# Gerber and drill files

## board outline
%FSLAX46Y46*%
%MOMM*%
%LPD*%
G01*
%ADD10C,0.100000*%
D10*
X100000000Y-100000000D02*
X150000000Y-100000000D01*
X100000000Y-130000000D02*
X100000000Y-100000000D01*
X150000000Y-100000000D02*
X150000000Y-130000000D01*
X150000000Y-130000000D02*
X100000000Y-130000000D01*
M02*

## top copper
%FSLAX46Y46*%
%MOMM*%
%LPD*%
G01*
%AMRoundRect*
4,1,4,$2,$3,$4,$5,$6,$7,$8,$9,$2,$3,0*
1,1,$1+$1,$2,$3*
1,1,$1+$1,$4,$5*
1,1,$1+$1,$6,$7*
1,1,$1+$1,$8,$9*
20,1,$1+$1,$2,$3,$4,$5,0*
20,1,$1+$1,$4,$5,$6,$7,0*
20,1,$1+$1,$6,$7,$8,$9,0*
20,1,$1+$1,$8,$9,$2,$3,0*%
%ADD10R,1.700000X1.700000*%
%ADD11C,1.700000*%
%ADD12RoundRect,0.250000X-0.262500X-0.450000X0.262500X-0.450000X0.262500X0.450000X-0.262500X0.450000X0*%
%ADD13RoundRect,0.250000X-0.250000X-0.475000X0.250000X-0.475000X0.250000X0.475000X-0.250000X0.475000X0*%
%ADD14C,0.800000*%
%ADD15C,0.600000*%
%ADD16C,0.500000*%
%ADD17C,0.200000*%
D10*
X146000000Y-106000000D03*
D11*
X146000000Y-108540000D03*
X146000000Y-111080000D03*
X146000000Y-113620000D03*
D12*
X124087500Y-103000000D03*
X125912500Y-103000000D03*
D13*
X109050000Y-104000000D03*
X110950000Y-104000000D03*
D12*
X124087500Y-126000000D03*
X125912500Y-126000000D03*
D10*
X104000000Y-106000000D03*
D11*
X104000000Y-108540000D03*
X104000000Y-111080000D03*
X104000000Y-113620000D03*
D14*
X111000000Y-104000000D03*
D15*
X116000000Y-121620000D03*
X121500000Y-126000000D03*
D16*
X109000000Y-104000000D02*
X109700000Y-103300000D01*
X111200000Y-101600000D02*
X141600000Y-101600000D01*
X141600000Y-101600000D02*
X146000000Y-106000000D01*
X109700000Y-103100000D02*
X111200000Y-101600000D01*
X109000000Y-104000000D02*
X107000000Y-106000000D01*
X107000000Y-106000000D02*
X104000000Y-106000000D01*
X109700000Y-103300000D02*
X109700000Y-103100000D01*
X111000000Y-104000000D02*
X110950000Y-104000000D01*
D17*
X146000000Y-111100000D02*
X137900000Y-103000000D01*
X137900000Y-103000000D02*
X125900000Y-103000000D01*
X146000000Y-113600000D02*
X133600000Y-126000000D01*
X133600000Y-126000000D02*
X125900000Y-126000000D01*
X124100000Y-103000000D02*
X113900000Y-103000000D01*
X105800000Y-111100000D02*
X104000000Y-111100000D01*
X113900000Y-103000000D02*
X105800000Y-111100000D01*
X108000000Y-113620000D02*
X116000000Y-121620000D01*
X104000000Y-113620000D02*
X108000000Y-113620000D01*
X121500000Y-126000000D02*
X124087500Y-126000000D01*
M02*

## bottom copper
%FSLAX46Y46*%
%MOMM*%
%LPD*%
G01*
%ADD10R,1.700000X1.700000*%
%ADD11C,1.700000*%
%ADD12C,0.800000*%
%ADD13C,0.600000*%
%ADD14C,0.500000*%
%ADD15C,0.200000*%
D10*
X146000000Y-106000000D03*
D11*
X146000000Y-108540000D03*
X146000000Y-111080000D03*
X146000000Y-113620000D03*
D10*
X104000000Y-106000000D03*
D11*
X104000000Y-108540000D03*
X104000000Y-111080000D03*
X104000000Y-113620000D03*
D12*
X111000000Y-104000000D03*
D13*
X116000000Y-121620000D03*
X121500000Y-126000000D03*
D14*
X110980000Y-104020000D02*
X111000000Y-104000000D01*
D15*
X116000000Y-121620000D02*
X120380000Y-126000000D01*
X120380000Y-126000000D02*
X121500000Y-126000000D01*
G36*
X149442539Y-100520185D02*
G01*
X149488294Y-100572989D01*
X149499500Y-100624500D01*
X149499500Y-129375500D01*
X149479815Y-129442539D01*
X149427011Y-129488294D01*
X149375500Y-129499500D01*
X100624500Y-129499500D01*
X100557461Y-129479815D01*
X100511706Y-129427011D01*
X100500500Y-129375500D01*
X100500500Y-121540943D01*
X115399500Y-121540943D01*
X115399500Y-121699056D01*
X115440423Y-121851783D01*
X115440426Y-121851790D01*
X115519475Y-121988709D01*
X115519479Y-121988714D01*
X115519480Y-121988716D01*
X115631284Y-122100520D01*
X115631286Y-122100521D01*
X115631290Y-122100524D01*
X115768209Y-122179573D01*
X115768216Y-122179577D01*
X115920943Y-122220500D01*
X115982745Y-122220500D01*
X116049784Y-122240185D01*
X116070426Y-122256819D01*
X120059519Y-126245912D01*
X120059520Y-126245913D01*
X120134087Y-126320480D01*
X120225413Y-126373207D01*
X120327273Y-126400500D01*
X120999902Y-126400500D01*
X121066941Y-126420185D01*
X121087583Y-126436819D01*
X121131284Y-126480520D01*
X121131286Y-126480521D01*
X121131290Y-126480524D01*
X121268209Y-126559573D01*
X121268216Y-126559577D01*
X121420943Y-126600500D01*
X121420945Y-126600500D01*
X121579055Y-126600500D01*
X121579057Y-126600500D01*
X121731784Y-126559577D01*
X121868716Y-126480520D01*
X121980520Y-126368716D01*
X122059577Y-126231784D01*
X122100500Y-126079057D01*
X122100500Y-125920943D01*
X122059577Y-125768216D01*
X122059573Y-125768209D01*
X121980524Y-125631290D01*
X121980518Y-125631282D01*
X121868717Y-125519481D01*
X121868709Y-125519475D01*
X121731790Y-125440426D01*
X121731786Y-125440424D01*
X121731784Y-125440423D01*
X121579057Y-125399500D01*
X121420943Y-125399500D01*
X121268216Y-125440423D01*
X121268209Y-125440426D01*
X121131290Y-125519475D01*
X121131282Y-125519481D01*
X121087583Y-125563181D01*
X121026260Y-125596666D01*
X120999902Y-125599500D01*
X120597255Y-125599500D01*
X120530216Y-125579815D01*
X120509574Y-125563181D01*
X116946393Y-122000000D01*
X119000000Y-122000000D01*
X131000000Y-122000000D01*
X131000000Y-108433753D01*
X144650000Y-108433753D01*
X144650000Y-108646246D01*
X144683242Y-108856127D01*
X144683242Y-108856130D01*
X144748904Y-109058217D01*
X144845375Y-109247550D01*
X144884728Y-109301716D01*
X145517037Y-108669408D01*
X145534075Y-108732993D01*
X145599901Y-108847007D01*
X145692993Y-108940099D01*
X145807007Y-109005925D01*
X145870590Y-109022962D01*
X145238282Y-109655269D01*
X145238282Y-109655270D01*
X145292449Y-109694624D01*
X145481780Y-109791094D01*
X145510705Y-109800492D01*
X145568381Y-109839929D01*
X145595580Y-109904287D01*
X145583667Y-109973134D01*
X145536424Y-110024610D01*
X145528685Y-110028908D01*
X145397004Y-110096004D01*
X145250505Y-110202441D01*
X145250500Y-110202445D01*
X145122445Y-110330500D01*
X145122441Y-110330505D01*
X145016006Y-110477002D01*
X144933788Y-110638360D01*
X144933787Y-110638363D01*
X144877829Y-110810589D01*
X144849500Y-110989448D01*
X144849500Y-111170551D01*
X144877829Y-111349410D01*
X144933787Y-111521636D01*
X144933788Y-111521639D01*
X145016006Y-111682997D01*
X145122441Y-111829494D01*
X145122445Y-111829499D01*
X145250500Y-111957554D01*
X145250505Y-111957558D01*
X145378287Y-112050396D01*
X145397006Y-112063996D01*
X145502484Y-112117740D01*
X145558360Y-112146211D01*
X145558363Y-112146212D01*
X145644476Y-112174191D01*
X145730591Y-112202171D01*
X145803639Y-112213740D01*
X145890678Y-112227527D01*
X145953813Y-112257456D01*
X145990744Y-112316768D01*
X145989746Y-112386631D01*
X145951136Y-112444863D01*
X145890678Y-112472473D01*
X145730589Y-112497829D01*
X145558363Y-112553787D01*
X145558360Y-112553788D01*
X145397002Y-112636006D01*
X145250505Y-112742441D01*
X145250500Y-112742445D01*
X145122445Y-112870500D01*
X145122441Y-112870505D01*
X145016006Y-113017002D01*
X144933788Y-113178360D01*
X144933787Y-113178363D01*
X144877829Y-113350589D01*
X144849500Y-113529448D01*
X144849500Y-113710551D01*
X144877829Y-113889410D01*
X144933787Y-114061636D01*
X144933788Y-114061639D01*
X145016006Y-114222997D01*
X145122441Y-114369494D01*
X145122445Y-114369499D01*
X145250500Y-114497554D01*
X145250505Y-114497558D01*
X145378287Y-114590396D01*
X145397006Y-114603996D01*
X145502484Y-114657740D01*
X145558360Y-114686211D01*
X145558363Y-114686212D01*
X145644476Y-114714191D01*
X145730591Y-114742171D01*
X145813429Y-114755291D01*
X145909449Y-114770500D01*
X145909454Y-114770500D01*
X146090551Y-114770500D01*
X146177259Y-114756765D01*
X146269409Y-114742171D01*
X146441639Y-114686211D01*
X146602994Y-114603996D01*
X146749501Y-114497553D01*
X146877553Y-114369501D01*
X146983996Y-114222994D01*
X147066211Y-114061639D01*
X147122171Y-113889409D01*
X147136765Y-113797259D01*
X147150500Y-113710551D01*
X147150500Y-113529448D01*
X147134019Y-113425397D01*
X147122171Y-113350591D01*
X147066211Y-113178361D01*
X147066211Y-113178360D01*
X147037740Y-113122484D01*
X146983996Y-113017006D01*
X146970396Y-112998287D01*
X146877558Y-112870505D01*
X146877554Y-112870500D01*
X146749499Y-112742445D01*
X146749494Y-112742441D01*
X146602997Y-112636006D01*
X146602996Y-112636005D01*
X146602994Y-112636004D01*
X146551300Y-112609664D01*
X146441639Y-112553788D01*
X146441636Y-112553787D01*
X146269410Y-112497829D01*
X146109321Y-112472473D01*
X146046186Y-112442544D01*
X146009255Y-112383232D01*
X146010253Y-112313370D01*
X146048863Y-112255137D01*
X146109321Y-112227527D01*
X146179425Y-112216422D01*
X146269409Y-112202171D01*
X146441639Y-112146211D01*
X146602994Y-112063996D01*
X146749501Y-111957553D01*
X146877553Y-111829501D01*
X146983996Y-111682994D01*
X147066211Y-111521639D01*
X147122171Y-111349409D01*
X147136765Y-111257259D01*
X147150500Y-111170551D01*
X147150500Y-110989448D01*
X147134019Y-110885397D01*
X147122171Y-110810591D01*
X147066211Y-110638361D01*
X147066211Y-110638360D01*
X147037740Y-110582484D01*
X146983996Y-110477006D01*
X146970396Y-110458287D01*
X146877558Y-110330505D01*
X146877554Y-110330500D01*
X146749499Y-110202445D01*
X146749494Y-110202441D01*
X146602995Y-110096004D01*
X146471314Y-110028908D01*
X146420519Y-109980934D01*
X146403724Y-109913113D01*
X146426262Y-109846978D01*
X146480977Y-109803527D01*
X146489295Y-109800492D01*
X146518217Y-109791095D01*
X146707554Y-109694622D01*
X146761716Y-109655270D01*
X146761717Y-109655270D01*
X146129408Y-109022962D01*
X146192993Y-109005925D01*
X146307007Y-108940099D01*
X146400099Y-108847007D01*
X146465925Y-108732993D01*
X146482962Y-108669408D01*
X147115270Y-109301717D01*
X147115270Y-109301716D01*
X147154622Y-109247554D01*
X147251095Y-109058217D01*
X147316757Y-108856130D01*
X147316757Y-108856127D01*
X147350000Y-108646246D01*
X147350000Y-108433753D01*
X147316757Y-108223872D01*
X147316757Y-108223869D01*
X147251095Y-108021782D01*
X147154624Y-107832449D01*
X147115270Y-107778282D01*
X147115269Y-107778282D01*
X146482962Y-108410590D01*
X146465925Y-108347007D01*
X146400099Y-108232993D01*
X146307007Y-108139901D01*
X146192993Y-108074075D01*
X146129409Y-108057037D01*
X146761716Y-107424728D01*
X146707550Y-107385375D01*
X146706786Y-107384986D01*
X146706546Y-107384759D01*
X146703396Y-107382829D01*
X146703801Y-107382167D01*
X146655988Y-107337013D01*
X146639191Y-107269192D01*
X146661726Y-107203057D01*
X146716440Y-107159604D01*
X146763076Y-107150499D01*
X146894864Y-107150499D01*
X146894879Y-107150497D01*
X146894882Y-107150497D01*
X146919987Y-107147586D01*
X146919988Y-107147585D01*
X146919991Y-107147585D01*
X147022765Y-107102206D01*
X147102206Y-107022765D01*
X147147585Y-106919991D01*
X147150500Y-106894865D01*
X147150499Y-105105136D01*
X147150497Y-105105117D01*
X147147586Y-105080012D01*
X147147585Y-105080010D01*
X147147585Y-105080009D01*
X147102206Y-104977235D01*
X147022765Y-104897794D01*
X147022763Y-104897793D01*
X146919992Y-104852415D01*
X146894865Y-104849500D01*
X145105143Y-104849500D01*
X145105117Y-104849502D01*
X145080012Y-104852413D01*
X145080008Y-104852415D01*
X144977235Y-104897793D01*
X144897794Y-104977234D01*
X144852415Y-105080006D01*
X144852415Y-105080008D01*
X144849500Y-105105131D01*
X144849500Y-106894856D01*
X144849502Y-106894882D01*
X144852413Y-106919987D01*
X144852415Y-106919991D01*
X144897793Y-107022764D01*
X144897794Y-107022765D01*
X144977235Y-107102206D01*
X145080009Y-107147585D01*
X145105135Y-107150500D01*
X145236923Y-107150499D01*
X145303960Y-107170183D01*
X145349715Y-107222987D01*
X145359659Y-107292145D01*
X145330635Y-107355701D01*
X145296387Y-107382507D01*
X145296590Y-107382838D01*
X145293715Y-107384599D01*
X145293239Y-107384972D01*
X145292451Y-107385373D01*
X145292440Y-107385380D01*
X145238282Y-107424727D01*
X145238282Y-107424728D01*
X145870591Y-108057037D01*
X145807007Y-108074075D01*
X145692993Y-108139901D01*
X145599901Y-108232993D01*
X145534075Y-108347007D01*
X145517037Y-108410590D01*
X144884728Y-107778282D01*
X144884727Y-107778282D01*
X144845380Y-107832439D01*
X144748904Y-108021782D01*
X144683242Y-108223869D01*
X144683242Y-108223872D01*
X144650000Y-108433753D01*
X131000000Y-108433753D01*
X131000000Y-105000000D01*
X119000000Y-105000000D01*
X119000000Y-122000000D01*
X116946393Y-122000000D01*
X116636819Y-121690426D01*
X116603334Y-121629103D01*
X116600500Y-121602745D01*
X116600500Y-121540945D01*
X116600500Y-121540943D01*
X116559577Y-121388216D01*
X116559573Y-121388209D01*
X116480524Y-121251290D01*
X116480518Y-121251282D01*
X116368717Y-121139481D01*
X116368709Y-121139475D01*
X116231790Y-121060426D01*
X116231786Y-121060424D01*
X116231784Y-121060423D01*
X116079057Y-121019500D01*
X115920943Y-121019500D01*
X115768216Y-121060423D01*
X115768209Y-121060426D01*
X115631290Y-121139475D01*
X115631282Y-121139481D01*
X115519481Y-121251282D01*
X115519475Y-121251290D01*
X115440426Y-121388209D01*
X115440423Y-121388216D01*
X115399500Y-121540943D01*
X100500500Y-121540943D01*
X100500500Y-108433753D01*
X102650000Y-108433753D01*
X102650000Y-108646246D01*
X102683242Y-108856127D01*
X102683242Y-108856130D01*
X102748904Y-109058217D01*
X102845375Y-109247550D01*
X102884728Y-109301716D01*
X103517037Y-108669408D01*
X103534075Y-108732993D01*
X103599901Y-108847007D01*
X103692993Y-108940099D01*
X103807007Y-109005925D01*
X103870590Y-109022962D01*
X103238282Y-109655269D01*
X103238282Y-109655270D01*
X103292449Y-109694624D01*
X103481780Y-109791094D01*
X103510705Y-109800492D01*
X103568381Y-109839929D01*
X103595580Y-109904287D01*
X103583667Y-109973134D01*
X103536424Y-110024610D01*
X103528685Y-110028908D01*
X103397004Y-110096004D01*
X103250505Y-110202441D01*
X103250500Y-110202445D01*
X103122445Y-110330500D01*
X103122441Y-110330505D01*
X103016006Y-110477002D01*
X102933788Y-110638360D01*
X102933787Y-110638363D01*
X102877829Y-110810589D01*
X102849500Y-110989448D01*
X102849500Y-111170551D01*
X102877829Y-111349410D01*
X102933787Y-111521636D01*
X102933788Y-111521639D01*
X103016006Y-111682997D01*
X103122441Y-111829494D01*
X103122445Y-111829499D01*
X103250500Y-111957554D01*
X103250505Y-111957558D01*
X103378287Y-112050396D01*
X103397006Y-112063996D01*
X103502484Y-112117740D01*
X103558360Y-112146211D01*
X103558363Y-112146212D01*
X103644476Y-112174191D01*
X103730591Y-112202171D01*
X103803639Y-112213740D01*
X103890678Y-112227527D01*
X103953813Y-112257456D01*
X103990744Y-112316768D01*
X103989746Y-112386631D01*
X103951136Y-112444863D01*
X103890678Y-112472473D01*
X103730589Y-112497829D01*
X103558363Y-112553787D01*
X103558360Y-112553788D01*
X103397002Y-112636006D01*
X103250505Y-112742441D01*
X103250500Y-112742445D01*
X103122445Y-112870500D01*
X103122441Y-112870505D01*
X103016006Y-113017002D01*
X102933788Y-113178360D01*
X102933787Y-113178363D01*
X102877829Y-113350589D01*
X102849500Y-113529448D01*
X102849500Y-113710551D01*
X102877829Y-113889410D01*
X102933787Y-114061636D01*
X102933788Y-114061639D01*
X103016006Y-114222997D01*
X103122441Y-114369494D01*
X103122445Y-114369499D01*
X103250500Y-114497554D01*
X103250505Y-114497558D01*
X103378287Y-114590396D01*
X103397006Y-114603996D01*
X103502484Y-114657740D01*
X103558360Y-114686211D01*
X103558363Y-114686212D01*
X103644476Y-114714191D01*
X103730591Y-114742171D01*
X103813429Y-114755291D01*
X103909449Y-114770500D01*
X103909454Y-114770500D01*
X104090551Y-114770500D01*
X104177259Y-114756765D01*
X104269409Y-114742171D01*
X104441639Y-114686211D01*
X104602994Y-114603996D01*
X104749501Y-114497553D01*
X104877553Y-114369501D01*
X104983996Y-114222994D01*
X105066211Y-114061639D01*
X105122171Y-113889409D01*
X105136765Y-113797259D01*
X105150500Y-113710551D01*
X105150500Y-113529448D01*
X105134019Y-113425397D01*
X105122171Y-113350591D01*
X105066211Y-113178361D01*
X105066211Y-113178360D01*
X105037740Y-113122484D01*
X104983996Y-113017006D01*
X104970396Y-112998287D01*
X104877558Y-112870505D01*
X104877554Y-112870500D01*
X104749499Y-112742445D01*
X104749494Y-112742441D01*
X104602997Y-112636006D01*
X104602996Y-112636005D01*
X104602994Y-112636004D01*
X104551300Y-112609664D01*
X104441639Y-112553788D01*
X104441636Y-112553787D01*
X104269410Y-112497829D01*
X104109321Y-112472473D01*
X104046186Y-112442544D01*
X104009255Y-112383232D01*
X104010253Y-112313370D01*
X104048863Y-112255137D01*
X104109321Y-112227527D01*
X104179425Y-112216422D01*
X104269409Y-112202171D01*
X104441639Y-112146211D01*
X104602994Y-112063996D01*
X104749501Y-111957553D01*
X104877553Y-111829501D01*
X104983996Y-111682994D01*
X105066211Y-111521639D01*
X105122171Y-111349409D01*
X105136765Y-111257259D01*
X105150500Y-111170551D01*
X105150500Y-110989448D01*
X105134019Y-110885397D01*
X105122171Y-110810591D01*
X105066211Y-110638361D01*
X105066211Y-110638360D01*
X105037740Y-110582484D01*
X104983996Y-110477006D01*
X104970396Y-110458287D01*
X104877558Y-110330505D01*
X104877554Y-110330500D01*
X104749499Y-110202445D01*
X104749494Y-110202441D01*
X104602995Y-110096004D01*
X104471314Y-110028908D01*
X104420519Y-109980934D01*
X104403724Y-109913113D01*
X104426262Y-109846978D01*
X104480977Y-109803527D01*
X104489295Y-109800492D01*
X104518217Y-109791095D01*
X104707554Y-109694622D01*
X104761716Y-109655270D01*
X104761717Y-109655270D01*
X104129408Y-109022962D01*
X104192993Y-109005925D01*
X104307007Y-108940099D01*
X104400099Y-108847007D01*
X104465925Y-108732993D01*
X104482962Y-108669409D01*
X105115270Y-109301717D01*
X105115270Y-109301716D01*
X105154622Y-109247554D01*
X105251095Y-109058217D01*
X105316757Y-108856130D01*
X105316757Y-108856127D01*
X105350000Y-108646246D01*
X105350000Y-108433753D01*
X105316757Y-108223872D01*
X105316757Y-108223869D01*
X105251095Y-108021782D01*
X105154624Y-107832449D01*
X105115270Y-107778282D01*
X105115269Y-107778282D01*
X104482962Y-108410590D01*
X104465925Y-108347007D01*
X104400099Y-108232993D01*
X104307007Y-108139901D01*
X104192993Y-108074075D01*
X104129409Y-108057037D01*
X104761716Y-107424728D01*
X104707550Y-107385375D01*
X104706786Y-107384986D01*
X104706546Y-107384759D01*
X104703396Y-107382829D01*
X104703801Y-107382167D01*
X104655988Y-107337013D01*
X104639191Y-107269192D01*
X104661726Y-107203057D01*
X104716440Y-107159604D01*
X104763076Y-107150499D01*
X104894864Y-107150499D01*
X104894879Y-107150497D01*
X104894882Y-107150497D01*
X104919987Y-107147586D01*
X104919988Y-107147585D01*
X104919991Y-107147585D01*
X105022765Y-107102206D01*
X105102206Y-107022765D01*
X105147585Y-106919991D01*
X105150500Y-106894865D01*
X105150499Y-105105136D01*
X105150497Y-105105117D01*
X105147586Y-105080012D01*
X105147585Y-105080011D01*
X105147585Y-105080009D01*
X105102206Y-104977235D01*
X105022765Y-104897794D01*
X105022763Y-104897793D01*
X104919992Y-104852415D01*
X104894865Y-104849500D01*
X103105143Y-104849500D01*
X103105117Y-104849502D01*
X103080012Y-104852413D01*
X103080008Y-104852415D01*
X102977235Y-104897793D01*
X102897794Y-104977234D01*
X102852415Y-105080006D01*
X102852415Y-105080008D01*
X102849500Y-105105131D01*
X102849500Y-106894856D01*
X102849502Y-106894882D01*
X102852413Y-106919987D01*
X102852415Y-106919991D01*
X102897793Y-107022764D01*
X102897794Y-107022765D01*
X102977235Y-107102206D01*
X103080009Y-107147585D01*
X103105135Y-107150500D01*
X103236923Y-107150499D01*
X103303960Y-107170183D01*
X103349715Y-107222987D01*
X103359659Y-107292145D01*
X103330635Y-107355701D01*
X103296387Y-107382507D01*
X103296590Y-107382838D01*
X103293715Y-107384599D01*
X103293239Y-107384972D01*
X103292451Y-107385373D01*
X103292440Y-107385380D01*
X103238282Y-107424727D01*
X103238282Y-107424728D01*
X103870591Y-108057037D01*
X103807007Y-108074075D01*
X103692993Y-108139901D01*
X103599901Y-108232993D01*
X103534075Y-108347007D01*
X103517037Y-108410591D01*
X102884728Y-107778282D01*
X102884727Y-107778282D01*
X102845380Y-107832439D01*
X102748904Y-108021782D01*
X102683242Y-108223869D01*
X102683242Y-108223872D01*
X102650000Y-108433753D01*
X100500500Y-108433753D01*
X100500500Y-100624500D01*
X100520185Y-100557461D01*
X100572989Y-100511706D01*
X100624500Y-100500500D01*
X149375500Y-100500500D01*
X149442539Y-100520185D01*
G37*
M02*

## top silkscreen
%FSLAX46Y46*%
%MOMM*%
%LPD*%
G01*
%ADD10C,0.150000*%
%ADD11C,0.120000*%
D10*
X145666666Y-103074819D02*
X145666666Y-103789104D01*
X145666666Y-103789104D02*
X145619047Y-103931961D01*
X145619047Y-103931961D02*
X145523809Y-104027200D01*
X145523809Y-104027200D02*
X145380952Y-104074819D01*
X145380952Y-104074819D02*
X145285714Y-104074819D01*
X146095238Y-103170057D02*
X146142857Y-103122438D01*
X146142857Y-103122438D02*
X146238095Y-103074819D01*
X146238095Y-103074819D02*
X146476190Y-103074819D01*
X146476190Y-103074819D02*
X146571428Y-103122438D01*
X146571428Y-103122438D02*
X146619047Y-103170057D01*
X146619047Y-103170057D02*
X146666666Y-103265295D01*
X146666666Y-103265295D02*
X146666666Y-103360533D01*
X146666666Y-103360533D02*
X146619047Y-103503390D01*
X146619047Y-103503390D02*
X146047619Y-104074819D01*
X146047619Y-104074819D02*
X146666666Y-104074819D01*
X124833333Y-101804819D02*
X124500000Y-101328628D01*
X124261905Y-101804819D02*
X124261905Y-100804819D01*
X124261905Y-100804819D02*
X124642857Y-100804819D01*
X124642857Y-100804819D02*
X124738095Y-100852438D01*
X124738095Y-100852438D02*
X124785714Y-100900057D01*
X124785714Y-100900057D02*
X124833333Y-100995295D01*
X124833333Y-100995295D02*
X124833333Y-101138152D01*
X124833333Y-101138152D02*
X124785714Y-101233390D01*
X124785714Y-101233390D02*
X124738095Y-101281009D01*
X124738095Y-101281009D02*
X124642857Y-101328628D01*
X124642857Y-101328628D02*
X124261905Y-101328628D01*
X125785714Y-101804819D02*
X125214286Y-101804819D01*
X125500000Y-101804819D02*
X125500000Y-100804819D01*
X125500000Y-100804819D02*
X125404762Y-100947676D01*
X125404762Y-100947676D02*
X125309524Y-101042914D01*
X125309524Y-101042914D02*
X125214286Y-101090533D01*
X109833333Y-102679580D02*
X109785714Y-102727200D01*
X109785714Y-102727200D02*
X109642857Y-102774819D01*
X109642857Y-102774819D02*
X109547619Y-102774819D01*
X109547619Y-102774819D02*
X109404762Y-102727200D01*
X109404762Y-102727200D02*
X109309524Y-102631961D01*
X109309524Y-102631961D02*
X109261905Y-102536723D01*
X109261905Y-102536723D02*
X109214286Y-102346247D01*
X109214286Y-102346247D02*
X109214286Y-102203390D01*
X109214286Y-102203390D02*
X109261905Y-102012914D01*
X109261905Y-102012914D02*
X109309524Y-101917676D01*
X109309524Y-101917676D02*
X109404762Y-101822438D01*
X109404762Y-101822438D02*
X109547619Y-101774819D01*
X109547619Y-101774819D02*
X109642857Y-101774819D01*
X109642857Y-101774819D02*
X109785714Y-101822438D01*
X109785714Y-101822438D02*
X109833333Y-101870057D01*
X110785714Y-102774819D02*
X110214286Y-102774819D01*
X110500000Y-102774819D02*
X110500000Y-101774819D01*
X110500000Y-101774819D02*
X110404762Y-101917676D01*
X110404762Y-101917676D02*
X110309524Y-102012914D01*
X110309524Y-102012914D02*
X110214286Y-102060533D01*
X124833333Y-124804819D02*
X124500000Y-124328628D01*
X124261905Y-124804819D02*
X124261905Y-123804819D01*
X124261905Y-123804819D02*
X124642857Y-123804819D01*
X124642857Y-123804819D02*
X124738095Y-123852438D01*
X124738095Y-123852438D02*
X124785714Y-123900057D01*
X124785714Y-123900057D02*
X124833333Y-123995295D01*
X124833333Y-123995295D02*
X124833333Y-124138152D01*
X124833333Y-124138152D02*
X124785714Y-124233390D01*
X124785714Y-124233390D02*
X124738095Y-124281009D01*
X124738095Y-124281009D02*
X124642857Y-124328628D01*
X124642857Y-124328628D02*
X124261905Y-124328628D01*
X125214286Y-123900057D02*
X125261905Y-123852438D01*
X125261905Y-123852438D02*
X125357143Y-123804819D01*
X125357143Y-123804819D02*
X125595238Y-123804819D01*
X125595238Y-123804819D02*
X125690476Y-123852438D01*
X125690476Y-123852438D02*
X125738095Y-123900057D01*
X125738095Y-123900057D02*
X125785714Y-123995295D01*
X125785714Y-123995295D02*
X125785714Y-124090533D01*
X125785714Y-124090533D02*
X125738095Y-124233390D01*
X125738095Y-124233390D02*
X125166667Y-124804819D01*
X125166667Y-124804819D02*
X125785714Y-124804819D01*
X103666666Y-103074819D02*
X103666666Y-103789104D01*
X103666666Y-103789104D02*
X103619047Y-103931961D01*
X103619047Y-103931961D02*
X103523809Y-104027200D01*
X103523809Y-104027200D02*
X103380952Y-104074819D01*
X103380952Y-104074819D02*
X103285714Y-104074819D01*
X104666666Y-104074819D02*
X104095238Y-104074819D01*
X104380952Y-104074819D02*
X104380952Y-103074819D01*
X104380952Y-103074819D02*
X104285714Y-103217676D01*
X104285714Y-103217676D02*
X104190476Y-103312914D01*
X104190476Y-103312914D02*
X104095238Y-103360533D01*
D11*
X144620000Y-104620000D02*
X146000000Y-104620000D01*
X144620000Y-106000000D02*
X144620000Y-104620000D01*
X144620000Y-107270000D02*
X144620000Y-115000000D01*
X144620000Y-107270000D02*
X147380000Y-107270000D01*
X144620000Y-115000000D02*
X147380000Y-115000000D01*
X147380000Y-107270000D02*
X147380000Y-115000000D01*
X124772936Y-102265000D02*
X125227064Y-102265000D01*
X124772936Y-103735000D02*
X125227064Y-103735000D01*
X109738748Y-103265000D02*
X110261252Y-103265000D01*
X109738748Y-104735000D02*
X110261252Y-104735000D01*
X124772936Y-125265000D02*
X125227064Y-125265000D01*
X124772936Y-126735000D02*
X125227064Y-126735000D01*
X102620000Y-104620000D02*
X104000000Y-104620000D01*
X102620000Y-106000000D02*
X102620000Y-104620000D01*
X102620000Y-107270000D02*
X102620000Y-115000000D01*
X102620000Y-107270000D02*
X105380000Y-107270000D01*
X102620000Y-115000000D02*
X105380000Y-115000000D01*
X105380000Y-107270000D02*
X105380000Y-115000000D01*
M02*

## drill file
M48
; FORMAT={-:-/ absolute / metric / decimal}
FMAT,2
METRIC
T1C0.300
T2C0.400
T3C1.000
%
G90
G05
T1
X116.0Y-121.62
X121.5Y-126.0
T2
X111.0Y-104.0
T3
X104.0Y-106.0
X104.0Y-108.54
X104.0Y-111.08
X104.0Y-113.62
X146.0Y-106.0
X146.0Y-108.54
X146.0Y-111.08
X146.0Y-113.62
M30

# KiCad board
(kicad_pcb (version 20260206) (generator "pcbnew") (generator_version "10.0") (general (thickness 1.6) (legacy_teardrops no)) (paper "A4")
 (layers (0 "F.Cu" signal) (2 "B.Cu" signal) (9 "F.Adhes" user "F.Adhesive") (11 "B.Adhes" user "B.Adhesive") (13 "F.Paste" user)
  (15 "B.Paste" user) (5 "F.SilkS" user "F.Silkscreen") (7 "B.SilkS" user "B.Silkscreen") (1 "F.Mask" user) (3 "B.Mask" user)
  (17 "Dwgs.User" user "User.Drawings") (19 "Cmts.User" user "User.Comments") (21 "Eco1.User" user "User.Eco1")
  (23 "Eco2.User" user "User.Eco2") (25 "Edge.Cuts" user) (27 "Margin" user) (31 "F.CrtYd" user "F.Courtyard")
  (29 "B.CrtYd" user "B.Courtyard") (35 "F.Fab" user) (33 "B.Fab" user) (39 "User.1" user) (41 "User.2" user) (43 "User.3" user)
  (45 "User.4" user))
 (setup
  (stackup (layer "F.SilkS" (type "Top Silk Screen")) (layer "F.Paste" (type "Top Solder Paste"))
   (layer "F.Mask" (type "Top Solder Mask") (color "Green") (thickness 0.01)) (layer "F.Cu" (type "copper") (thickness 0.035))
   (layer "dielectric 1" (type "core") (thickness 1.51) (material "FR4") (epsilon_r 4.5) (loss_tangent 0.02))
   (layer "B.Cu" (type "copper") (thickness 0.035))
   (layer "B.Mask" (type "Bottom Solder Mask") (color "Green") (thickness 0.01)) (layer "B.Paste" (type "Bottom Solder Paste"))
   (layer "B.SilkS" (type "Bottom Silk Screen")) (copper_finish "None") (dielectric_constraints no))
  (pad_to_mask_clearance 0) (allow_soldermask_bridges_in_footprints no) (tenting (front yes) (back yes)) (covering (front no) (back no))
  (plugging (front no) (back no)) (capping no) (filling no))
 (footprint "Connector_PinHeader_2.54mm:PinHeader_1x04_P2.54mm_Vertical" (layer "F.Cu") (at 146 106)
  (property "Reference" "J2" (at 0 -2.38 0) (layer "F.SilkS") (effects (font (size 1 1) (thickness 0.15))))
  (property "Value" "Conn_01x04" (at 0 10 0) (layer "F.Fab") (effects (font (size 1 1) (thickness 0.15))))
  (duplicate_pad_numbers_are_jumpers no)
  (fp_line (start -1.38 -1.38) (end 0 -1.38) (stroke (width 0.12) (type solid)) (layer "F.SilkS"))
  (fp_line (start -1.38 0) (end -1.38 -1.38) (stroke (width 0.12) (type solid)) (layer "F.SilkS"))
  (fp_line (start -1.38 1.27) (end -1.38 9) (stroke (width 0.12) (type solid)) (layer "F.SilkS"))
  (fp_line (start -1.38 1.27) (end 1.38 1.27) (stroke (width 0.12) (type solid)) (layer "F.SilkS"))
  (fp_line (start -1.38 9) (end 1.38 9) (stroke (width 0.12) (type solid)) (layer "F.SilkS"))
  (fp_line (start 1.38 1.27) (end 1.38 9) (stroke (width 0.12) (type solid)) (layer "F.SilkS"))
  (pad "1" thru_hole rect (at 0 0) (size 1.7 1.7) (drill 1) (layers "*.Cu" "*.Mask") (remove_unused_layers no) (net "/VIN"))
  (pad "2" thru_hole circle (at 0 2.54) (size 1.7 1.7) (drill 1) (layers "*.Cu" "*.Mask") (remove_unused_layers no) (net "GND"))
  (pad "3" thru_hole circle (at 0 5.08) (size 1.7 1.7) (drill 1) (layers "*.Cu" "*.Mask") (remove_unused_layers no) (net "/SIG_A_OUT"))
  (pad "4" thru_hole circle (at 0 7.62) (size 1.7 1.7) (drill 1) (layers "*.Cu" "*.Mask") (remove_unused_layers no) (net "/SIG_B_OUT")))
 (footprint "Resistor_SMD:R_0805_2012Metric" (layer "F.Cu") (at 125 103)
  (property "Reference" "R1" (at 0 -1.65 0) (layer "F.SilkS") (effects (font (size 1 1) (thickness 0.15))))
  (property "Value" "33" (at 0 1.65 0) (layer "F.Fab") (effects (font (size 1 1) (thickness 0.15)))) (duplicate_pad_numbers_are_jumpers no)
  (fp_line (start -0.227064 -0.735) (end 0.227064 -0.735) (stroke (width 0.12) (type solid)) (layer "F.SilkS"))
  (fp_line (start -0.227064 0.735) (end 0.227064 0.735) (stroke (width 0.12) (type solid)) (layer "F.SilkS"))
  (pad "1" smd roundrect (at -0.9125 0) (size 1.025 1.4) (layers "F.Cu" "F.Mask" "F.Paste") (roundrect_rratio 0.243902) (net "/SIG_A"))
  (pad "2" smd roundrect (at 0.9125 0) (size 1.025 1.4) (layers "F.Cu" "F.Mask" "F.Paste") (roundrect_rratio 0.243902) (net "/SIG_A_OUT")))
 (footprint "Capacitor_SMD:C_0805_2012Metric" (layer "F.Cu") (at 110 104)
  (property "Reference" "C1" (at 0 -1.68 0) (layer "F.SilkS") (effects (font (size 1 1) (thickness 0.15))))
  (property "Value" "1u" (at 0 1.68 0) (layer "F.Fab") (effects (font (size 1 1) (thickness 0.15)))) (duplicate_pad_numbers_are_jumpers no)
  (fp_line (start -0.261252 -0.735) (end 0.261252 -0.735) (stroke (width 0.12) (type solid)) (layer "F.SilkS"))
  (fp_line (start -0.261252 0.735) (end 0.261252 0.735) (stroke (width 0.12) (type solid)) (layer "F.SilkS"))
  (pad "1" smd roundrect (at -0.95 0) (size 1 1.45) (layers "F.Cu" "F.Mask" "F.Paste") (roundrect_rratio 0.25) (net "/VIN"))
  (pad "2" smd roundrect (at 0.95 0) (size 1 1.45) (layers "F.Cu" "F.Mask" "F.Paste") (roundrect_rratio 0.25) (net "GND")))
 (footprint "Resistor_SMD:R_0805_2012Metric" (layer "F.Cu") (at 125 126)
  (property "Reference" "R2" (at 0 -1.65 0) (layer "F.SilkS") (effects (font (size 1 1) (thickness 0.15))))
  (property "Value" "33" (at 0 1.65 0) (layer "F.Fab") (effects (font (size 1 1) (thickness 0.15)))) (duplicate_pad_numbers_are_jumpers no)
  (fp_line (start -0.227064 -0.735) (end 0.227064 -0.735) (stroke (width 0.12) (type solid)) (layer "F.SilkS"))
  (fp_line (start -0.227064 0.735) (end 0.227064 0.735) (stroke (width 0.12) (type solid)) (layer "F.SilkS"))
  (pad "1" smd roundrect (at -0.9125 0) (size 1.025 1.4) (layers "F.Cu" "F.Mask" "F.Paste") (roundrect_rratio 0.243902) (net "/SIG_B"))
  (pad "2" smd roundrect (at 0.9125 0) (size 1.025 1.4) (layers "F.Cu" "F.Mask" "F.Paste") (roundrect_rratio 0.243902) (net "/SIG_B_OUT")))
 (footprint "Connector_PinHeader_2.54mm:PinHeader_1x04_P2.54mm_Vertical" (layer "F.Cu") (at 104 106)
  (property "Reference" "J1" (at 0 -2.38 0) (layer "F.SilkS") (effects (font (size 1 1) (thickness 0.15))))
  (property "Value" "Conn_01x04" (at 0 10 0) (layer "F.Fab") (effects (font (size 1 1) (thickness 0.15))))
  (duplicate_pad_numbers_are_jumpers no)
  (fp_line (start -1.38 -1.38) (end 0 -1.38) (stroke (width 0.12) (type solid)) (layer "F.SilkS"))
  (fp_line (start -1.38 0) (end -1.38 -1.38) (stroke (width 0.12) (type solid)) (layer "F.SilkS"))
  (fp_line (start -1.38 1.27) (end -1.38 9) (stroke (width 0.12) (type solid)) (layer "F.SilkS"))
  (fp_line (start -1.38 1.27) (end 1.38 1.27) (stroke (width 0.12) (type solid)) (layer "F.SilkS"))
  (fp_line (start -1.38 9) (end 1.38 9) (stroke (width 0.12) (type solid)) (layer "F.SilkS"))
  (fp_line (start 1.38 1.27) (end 1.38 9) (stroke (width 0.12) (type solid)) (layer "F.SilkS"))
  (pad "1" thru_hole rect (at 0 0) (size 1.7 1.7) (drill 1) (layers "*.Cu" "*.Mask") (remove_unused_layers no) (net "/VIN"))
  (pad "2" thru_hole circle (at 0 2.54) (size 1.7 1.7) (drill 1) (layers "*.Cu" "*.Mask") (remove_unused_layers no) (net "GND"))
  (pad "3" thru_hole circle (at 0 5.08) (size 1.7 1.7) (drill 1) (layers "*.Cu" "*.Mask") (remove_unused_layers no) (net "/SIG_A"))
  (pad "4" thru_hole circle (at 0 7.62) (size 1.7 1.7) (drill 1) (layers "*.Cu" "*.Mask") (remove_unused_layers no) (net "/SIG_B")))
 (gr_line (start 100 100) (end 150 100) (stroke (width 0.1) (type default)) (layer "Edge.Cuts"))
 (gr_line (start 100 130) (end 100 100) (stroke (width 0.1) (type default)) (layer "Edge.Cuts"))
 (gr_line (start 150 100) (end 150 130) (stroke (width 0.1) (type default)) (layer "Edge.Cuts"))
 (gr_line (start 150 130) (end 100 130) (stroke (width 0.1) (type default)) (layer "Edge.Cuts"))
 (segment (start 109 104) (end 109.7 103.3) (width 0.5) (layer "F.Cu") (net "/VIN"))
 (segment (start 111.2 101.6) (end 141.6 101.6) (width 0.5) (layer "F.Cu") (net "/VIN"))
 (segment (start 141.6 101.6) (end 146 106) (width 0.5) (layer "F.Cu") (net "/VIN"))
 (segment (start 109.7 103.1) (end 111.2 101.6) (width 0.5) (layer "F.Cu") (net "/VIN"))
 (segment (start 109 104) (end 107 106) (width 0.5) (layer "F.Cu") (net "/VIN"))
 (segment (start 107 106) (end 104 106) (width 0.5) (layer "F.Cu") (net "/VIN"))
 (segment (start 109.7 103.3) (end 109.7 103.1) (width 0.5) (layer "F.Cu") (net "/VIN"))
 (segment (start 111 104) (end 110.95 104) (width 0.5) (layer "F.Cu") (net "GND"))
 (via (at 111 104) (size 0.8) (drill 0.4) (layers "F.Cu" "B.Cu") (capping yes) (filling yes) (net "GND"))
 (segment (start 110.98 104.02) (end 111 104) (width 0.5) (layer "B.Cu") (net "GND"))
 (segment (start 146 111.1) (end 137.9 103) (width 0.2) (layer "F.Cu") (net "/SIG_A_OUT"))
 (segment (start 137.9 103) (end 125.9 103) (width 0.2) (layer "F.Cu") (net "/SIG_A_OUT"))
 (segment (start 146 113.6) (end 133.6 126) (width 0.2) (layer "F.Cu") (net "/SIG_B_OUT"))
 (segment (start 133.6 126) (end 125.9 126) (width 0.2) (layer "F.Cu") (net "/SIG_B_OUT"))
 (segment (start 124.1 103) (end 113.9 103) (width 0.2) (layer "F.Cu") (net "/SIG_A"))
 (segment (start 105.8 111.1) (end 104 111.1) (width 0.2) (layer "F.Cu") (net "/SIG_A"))
 (segment (start 113.9 103) (end 105.8 111.1) (width 0.2) (layer "F.Cu") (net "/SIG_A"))
 (segment (start 108 113.62) (end 116 121.62) (width 0.2) (locked yes) (layer "F.Cu") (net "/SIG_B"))
 (segment (start 104 113.62) (end 108 113.62) (width 0.2) (locked yes) (layer "F.Cu") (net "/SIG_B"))
 (segment (start 121.5 126) (end 124.0875 126) (width 0.2) (locked yes) (layer "F.Cu") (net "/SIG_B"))
 (via (at 116 121.62) (size 0.6) (drill 0.3) (layers "F.Cu" "B.Cu") (locked yes) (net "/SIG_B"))
 (via (at 121.5 126) (size 0.6) (drill 0.3) (layers "F.Cu" "B.Cu") (locked yes) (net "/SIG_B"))
 (segment (start 116 121.62) (end 120.38 126) (width 0.2) (locked yes) (layer "B.Cu") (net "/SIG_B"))
 (segment (start 120.38 126) (end 121.5 126) (width 0.2) (locked yes) (layer "B.Cu") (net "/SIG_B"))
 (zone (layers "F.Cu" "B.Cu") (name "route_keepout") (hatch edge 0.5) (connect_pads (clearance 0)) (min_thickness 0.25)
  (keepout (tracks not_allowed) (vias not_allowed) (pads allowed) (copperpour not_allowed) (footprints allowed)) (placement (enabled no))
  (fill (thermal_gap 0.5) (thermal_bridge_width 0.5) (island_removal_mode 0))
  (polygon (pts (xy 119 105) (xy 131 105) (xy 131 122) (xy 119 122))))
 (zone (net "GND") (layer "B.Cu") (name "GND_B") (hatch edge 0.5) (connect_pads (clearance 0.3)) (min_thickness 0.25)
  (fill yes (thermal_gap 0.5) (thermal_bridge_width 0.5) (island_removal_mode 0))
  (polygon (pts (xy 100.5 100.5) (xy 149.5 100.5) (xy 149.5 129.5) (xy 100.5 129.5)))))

